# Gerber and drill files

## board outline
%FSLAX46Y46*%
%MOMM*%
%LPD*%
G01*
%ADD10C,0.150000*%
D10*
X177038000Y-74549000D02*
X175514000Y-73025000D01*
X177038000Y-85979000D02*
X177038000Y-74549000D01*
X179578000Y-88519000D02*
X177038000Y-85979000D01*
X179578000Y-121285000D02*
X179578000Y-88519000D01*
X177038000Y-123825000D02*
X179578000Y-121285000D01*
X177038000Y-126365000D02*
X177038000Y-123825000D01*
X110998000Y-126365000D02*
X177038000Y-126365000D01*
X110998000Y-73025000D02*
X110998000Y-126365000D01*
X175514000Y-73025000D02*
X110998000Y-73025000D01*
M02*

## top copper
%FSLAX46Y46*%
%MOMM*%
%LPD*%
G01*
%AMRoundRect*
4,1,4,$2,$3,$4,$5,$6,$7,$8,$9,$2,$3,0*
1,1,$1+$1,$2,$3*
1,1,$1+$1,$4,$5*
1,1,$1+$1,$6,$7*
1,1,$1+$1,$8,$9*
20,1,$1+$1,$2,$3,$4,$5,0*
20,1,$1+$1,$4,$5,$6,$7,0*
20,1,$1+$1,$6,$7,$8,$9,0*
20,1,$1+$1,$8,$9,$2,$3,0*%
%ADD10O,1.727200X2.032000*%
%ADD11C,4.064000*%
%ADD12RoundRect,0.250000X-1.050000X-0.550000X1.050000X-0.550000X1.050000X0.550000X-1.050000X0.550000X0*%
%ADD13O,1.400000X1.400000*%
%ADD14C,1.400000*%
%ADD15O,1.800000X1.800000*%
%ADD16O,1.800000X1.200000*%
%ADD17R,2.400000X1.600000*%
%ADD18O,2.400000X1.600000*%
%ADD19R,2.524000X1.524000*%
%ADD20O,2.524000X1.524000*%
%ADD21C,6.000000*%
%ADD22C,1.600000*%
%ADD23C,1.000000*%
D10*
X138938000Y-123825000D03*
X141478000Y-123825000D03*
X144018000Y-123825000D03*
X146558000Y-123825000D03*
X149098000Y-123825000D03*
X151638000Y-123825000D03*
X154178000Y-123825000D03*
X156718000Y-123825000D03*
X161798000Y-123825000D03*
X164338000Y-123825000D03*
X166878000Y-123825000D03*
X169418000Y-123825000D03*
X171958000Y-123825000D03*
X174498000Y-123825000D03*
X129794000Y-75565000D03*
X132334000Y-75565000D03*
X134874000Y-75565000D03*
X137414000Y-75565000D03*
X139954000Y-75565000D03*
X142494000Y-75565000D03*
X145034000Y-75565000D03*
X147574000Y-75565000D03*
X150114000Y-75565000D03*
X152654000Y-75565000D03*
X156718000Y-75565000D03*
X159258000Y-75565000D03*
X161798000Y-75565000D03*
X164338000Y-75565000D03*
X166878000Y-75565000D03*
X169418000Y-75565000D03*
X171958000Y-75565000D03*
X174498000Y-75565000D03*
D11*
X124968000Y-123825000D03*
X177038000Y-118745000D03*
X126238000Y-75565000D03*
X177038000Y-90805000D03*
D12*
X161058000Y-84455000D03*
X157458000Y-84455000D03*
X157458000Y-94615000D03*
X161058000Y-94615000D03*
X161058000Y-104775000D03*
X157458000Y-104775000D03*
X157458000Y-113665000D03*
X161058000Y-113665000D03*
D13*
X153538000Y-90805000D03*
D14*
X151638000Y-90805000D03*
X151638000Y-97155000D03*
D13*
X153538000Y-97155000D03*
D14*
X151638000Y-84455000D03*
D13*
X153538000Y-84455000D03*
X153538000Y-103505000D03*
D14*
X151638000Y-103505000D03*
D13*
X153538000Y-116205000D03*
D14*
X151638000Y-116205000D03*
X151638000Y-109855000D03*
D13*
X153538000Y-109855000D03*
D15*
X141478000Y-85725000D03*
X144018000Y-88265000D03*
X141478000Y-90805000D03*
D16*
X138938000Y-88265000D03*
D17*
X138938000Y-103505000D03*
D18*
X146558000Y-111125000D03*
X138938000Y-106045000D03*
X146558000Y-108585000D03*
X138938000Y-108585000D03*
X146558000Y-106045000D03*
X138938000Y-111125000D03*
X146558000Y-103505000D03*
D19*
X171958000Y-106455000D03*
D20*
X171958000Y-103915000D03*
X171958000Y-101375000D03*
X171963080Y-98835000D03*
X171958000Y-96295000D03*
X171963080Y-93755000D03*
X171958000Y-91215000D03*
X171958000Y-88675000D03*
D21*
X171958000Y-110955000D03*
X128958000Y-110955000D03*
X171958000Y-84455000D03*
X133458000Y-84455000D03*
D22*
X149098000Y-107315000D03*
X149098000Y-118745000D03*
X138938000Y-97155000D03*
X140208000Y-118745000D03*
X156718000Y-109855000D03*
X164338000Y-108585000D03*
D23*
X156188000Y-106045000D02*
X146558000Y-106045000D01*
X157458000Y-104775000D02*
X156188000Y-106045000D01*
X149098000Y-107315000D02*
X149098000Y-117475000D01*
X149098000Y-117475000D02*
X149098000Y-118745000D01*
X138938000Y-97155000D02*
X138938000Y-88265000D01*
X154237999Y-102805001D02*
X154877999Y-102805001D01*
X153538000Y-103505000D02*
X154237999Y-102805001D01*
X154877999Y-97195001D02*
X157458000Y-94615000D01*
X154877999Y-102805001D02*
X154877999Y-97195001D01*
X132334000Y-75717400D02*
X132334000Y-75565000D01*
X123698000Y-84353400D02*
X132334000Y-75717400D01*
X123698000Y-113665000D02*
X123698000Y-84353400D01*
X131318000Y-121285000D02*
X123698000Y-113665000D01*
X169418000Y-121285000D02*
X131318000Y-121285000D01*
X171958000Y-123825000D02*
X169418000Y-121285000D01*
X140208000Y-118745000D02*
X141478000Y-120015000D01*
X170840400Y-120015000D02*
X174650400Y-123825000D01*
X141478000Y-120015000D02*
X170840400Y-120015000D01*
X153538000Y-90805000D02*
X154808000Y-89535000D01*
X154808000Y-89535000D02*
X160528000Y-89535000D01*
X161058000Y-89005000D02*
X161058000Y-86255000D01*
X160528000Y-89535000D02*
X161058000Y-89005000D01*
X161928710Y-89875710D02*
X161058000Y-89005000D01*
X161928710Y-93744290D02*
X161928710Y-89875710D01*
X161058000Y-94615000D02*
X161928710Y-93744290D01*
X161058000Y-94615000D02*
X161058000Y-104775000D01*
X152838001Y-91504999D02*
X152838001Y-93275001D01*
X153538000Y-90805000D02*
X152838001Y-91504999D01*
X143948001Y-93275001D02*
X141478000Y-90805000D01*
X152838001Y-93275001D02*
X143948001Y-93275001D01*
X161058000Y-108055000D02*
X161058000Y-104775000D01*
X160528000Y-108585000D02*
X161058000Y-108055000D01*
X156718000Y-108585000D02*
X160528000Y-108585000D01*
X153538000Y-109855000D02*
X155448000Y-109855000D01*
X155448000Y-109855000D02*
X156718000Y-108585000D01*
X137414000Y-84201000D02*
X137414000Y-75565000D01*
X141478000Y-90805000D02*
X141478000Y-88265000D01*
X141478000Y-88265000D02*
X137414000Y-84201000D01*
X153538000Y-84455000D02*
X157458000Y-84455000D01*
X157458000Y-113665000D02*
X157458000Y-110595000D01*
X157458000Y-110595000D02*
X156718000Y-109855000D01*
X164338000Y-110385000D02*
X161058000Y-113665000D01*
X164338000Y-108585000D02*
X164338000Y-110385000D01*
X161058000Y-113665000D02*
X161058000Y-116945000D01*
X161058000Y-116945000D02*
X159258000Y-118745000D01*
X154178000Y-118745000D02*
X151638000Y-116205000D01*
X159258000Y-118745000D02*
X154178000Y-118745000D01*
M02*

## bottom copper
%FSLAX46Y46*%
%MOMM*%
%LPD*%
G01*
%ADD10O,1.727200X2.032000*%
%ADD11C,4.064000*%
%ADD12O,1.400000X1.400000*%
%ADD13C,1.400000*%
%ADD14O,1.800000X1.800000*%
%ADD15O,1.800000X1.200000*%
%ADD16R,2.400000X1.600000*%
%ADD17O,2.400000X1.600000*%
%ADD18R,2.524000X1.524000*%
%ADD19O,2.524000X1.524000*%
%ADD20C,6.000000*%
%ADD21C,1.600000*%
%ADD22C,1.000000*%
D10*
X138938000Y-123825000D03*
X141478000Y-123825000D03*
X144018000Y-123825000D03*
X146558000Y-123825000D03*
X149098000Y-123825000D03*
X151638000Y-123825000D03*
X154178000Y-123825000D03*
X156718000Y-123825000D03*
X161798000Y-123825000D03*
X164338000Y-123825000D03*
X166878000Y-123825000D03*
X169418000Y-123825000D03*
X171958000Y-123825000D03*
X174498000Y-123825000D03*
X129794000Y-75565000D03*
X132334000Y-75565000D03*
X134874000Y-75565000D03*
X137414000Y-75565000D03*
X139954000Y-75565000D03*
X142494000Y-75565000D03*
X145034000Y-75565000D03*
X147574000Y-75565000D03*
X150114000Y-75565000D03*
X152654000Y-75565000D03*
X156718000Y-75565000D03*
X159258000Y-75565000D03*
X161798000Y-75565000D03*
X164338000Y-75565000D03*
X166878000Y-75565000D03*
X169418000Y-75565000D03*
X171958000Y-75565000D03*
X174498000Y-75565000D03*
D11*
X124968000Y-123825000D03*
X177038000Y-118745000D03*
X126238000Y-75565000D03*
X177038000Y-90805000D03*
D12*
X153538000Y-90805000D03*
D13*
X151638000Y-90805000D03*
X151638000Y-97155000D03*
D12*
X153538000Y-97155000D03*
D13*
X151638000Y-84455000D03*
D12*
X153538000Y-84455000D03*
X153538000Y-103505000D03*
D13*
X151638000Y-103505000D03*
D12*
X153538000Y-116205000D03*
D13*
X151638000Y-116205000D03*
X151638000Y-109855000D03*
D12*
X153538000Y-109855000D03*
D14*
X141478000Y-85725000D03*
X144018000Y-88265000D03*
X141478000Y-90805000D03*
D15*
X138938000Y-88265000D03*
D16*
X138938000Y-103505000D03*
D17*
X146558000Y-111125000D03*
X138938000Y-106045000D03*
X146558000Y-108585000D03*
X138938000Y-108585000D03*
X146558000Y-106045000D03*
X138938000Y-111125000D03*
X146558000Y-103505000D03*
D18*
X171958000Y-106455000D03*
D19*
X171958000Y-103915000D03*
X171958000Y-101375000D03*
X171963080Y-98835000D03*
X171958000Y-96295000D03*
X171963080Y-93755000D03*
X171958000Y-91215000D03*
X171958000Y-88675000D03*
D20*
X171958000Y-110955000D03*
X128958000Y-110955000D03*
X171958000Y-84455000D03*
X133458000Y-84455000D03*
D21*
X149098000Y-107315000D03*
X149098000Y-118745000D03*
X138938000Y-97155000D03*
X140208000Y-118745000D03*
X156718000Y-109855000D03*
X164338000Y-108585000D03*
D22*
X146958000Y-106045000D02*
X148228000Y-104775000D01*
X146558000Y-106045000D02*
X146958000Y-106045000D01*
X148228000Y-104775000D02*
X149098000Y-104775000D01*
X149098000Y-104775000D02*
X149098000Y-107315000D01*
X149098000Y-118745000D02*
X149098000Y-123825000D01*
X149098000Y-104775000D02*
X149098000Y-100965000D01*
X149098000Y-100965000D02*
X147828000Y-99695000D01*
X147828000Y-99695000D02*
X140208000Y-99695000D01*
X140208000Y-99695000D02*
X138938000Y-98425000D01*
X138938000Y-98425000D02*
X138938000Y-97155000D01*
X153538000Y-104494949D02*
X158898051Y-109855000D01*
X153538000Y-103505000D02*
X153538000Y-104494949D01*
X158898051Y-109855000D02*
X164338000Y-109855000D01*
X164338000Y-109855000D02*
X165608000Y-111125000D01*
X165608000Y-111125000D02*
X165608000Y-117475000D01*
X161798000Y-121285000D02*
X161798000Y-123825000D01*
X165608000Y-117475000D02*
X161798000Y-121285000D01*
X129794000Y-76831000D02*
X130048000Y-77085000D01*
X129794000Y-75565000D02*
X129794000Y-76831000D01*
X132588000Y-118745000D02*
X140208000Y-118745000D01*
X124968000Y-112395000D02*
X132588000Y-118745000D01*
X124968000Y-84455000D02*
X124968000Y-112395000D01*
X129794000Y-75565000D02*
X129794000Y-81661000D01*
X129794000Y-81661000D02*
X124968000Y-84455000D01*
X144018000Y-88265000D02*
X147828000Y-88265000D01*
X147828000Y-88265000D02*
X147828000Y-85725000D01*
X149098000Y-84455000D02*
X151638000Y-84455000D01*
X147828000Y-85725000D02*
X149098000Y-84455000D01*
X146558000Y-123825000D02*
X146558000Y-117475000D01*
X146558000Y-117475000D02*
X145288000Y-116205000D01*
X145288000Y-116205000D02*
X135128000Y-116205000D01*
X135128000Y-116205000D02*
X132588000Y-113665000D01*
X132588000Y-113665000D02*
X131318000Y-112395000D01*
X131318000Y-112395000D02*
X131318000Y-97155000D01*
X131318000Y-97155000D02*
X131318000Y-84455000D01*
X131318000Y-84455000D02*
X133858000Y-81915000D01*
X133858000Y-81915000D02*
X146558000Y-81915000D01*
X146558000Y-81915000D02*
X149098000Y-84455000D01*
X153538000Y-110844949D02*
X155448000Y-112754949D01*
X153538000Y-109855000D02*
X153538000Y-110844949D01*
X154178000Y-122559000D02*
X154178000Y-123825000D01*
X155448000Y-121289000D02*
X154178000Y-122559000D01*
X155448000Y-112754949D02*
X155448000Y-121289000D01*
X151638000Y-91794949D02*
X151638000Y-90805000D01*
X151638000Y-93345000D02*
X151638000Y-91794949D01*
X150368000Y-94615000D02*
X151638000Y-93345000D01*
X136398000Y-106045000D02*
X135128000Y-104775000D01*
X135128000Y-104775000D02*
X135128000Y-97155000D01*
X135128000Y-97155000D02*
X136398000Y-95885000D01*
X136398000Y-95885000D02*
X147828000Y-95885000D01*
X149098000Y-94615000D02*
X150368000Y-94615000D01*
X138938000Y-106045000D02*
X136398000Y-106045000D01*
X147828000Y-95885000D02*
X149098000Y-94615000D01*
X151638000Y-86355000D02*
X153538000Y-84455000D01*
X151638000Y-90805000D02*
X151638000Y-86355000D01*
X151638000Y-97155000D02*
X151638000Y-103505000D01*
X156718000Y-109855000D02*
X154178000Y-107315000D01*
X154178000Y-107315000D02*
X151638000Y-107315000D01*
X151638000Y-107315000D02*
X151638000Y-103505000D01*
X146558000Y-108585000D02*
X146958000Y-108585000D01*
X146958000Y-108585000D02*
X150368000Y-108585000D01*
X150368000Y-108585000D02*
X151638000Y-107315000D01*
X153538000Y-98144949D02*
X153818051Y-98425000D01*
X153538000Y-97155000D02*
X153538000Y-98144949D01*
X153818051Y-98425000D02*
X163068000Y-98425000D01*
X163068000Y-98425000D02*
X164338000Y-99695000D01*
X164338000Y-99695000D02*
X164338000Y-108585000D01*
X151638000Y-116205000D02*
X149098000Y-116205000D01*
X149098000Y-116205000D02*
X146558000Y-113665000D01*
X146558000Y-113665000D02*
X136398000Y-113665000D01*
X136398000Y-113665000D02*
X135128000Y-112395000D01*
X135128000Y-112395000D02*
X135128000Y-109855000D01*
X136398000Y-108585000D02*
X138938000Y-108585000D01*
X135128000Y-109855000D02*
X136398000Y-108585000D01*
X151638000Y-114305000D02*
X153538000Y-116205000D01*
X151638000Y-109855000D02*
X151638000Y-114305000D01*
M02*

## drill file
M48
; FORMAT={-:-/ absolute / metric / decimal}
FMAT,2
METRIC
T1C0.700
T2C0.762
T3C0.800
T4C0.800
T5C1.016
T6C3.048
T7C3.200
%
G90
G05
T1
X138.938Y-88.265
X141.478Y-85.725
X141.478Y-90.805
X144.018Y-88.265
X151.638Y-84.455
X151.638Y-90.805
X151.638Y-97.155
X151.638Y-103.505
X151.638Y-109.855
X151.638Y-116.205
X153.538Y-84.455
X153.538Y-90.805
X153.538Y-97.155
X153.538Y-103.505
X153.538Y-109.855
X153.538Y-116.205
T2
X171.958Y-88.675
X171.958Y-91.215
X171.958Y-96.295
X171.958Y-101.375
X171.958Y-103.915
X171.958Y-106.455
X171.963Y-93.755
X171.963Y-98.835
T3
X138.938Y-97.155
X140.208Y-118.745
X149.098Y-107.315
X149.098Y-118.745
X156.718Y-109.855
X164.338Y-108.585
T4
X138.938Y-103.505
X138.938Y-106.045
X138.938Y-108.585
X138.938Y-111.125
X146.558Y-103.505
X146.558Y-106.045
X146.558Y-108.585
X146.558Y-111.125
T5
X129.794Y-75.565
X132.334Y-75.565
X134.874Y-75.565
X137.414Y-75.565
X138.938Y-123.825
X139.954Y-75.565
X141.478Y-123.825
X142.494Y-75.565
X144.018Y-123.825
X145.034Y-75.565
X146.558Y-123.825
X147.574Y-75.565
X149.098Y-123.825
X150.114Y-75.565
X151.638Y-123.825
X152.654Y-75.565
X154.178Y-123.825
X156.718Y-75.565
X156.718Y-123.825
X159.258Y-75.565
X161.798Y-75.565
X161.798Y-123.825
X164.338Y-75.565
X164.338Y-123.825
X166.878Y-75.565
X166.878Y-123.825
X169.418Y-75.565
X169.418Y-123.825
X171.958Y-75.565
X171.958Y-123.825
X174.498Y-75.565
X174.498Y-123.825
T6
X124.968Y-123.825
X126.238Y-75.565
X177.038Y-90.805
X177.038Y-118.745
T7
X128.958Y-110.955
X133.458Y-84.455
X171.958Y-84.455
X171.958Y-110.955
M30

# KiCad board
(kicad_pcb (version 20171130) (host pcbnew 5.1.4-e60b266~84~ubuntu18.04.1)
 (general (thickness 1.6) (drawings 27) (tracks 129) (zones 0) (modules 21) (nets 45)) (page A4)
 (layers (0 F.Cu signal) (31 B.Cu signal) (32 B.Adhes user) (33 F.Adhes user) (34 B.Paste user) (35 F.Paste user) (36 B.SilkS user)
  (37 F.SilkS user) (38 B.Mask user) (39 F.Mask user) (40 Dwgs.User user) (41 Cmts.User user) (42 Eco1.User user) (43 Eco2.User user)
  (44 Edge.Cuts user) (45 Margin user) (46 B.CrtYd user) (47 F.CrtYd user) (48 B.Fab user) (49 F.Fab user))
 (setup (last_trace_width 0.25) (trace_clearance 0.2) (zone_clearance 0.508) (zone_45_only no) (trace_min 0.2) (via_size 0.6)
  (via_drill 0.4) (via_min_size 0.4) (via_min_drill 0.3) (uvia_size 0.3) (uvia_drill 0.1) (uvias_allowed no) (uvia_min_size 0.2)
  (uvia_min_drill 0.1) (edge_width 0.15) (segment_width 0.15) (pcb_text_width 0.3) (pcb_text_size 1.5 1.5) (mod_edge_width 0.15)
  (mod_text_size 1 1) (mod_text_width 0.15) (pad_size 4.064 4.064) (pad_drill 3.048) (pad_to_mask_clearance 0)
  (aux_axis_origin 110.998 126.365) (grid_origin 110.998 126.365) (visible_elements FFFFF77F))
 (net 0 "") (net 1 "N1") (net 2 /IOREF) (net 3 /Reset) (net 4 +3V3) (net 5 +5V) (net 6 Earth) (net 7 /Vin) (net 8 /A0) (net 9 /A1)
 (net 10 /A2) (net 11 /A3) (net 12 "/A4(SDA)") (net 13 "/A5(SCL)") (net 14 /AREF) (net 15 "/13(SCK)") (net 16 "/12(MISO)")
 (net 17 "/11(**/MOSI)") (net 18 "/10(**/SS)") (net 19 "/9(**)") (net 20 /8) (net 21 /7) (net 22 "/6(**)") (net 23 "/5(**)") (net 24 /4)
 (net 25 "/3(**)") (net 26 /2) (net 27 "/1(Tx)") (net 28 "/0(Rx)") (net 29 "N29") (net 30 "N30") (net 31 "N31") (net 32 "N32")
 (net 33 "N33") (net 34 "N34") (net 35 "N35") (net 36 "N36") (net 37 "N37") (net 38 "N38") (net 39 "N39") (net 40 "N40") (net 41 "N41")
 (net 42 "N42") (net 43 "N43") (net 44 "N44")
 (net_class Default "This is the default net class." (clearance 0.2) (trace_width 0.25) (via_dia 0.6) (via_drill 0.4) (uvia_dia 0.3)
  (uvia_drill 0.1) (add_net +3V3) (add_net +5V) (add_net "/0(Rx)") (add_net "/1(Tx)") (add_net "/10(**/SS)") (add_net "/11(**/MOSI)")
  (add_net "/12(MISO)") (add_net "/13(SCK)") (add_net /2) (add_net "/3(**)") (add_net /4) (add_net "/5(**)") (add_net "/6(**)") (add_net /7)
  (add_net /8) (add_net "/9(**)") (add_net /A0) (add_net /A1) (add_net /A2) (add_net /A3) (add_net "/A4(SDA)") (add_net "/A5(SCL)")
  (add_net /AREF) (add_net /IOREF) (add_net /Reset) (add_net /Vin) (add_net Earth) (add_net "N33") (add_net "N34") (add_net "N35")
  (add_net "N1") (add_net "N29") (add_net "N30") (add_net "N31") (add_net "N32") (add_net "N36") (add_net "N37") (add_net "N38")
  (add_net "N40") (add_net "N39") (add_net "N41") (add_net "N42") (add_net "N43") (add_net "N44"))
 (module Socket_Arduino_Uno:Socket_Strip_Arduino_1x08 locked (layer F.Cu) (at 138.938 123.825)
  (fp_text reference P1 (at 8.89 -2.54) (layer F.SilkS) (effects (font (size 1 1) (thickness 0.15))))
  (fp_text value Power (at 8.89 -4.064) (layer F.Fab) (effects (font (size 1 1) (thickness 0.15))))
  (pad 1 thru_hole oval (at 0 0) (size 1.7272 2.032) (drill 1.016) (layers *.Cu *.Mask F.SilkS) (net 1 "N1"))
  (pad 2 thru_hole oval (at 2.54 0) (size 1.7272 2.032) (drill 1.016) (layers *.Cu *.Mask F.SilkS) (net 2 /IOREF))
  (pad 3 thru_hole oval (at 5.08 0) (size 1.7272 2.032) (drill 1.016) (layers *.Cu *.Mask F.SilkS) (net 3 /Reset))
  (pad 4 thru_hole oval (at 7.62 0) (size 1.7272 2.032) (drill 1.016) (layers *.Cu *.Mask F.SilkS) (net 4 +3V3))
  (pad 5 thru_hole oval (at 10.16 0) (size 1.7272 2.032) (drill 1.016) (layers *.Cu *.Mask F.SilkS) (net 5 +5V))
  (pad 6 thru_hole oval (at 12.7 0) (size 1.7272 2.032) (drill 1.016) (layers *.Cu *.Mask F.SilkS) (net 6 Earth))
  (pad 7 thru_hole oval (at 15.24 0) (size 1.7272 2.032) (drill 1.016) (layers *.Cu *.Mask F.SilkS) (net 6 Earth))
  (pad 8 thru_hole oval (at 17.78 0) (size 1.7272 2.032) (drill 1.016) (layers *.Cu *.Mask F.SilkS) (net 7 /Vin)))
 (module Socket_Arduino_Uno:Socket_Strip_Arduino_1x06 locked (layer F.Cu) (at 161.798 123.825)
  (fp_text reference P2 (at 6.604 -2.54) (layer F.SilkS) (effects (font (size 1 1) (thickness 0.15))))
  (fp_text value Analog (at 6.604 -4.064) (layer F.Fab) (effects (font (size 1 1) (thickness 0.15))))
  (pad 1 thru_hole oval (at 0 0) (size 1.7272 2.032) (drill 1.016) (layers *.Cu *.Mask F.SilkS) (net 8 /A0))
  (pad 2 thru_hole oval (at 2.54 0) (size 1.7272 2.032) (drill 1.016) (layers *.Cu *.Mask F.SilkS) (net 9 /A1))
  (pad 3 thru_hole oval (at 5.08 0) (size 1.7272 2.032) (drill 1.016) (layers *.Cu *.Mask F.SilkS) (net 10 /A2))
  (pad 4 thru_hole oval (at 7.62 0) (size 1.7272 2.032) (drill 1.016) (layers *.Cu *.Mask F.SilkS) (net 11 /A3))
  (pad 5 thru_hole oval (at 10.16 0) (size 1.7272 2.032) (drill 1.016) (layers *.Cu *.Mask F.SilkS) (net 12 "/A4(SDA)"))
  (pad 6 thru_hole oval (at 12.7 0) (size 1.7272 2.032) (drill 1.016) (layers *.Cu *.Mask F.SilkS) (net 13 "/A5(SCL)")))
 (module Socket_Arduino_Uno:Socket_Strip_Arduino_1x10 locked (layer F.Cu) (at 129.794 75.565)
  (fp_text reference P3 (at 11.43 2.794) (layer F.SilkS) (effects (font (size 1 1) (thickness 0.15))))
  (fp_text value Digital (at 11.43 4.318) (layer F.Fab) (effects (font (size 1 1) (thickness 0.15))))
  (pad 1 thru_hole oval (at 0 0) (size 1.7272 2.032) (drill 1.016) (layers *.Cu *.Mask F.SilkS) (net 13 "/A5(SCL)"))
  (pad 2 thru_hole oval (at 2.54 0) (size 1.7272 2.032) (drill 1.016) (layers *.Cu *.Mask F.SilkS) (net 12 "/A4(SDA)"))
  (pad 3 thru_hole oval (at 5.08 0) (size 1.7272 2.032) (drill 1.016) (layers *.Cu *.Mask F.SilkS) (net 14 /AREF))
  (pad 4 thru_hole oval (at 7.62 0) (size 1.7272 2.032) (drill 1.016) (layers *.Cu *.Mask F.SilkS) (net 6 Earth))
  (pad 5 thru_hole oval (at 10.16 0) (size 1.7272 2.032) (drill 1.016) (layers *.Cu *.Mask F.SilkS) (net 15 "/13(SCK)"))
  (pad 6 thru_hole oval (at 12.7 0) (size 1.7272 2.032) (drill 1.016) (layers *.Cu *.Mask F.SilkS) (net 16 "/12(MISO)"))
  (pad 7 thru_hole oval (at 15.24 0) (size 1.7272 2.032) (drill 1.016) (layers *.Cu *.Mask F.SilkS) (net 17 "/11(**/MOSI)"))
  (pad 8 thru_hole oval (at 17.78 0) (size 1.7272 2.032) (drill 1.016) (layers *.Cu *.Mask F.SilkS) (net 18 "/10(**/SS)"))
  (pad 9 thru_hole oval (at 20.32 0) (size 1.7272 2.032) (drill 1.016) (layers *.Cu *.Mask F.SilkS) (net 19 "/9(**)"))
  (pad 10 thru_hole oval (at 22.86 0) (size 1.7272 2.032) (drill 1.016) (layers *.Cu *.Mask F.SilkS) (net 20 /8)))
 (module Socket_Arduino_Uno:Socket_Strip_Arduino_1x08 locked (layer F.Cu) (at 156.718 75.565)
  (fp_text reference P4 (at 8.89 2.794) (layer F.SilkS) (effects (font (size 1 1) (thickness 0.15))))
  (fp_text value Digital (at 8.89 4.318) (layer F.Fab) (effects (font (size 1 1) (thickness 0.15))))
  (pad 1 thru_hole oval (at 0 0) (size 1.7272 2.032) (drill 1.016) (layers *.Cu *.Mask F.SilkS) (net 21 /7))
  (pad 2 thru_hole oval (at 2.54 0) (size 1.7272 2.032) (drill 1.016) (layers *.Cu *.Mask F.SilkS) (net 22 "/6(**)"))
  (pad 3 thru_hole oval (at 5.08 0) (size 1.7272 2.032) (drill 1.016) (layers *.Cu *.Mask F.SilkS) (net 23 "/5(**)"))
  (pad 4 thru_hole oval (at 7.62 0) (size 1.7272 2.032) (drill 1.016) (layers *.Cu *.Mask F.SilkS) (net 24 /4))
  (pad 5 thru_hole oval (at 10.16 0) (size 1.7272 2.032) (drill 1.016) (layers *.Cu *.Mask F.SilkS) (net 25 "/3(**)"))
  (pad 6 thru_hole oval (at 12.7 0) (size 1.7272 2.032) (drill 1.016) (layers *.Cu *.Mask F.SilkS) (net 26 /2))
  (pad 7 thru_hole oval (at 15.24 0) (size 1.7272 2.032) (drill 1.016) (layers *.Cu *.Mask F.SilkS) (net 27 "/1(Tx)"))
  (pad 8 thru_hole oval (at 17.78 0) (size 1.7272 2.032) (drill 1.016) (layers *.Cu *.Mask F.SilkS) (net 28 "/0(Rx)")))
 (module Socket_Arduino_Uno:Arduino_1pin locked (layer F.Cu) (at 124.968 123.825)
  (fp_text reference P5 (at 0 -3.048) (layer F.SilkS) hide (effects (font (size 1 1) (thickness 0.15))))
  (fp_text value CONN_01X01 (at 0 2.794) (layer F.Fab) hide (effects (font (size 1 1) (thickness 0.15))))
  (pad 1 thru_hole circle (at 0 0) (size 4.064 4.064) (drill 3.048) (layers *.Cu *.Mask F.SilkS) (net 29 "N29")))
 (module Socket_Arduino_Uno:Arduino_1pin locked (layer F.Cu) (at 177.038 118.745)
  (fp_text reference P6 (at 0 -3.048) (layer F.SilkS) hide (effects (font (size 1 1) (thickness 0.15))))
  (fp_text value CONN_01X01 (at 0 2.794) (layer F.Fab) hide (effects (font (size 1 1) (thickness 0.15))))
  (pad 1 thru_hole circle (at 0 0) (size 4.064 4.064) (drill 3.048) (layers *.Cu *.Mask F.SilkS) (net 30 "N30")))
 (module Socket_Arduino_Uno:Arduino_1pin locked (layer F.Cu) (at 126.238 75.565)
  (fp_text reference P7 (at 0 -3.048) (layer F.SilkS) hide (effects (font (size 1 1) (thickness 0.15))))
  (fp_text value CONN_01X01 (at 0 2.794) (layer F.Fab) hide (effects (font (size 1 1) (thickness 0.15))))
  (pad 1 thru_hole circle (at 0 0) (size 4.064 4.064) (drill 3.048) (layers *.Cu *.Mask F.SilkS) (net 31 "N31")))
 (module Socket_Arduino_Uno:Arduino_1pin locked (layer F.Cu) (at 177.038 90.805)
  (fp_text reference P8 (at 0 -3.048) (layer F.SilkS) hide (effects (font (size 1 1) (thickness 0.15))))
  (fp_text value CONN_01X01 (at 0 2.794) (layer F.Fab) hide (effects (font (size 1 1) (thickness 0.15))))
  (pad 1 thru_hole circle (at 0 0) (size 4.064 4.064) (drill 3.048) (layers *.Cu *.Mask F.SilkS) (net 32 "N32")))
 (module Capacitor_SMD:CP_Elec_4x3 (layer F.Cu) (at 159.258 84.455)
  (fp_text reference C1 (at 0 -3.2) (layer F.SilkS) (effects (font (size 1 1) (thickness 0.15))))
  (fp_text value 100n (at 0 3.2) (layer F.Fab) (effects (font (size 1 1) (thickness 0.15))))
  (pad 2 smd roundrect (at 1.8 0) (size 2.6 1.6) (layers F.Cu F.Paste F.Mask) (roundrect_rratio 0.15625) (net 6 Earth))
  (pad 1 smd roundrect (at -1.8 0) (size 2.6 1.6) (layers F.Cu F.Paste F.Mask) (roundrect_rratio 0.15625) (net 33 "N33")))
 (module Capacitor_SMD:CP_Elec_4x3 (layer F.Cu) (at 159.258 94.615)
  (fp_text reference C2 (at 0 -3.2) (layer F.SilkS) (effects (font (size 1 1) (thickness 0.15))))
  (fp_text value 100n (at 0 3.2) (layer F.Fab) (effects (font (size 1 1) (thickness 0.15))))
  (pad 1 smd roundrect (at -1.8 0) (size 2.6 1.6) (layers F.Cu F.Paste F.Mask) (roundrect_rratio 0.15625) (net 8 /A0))
  (pad 2 smd roundrect (at 1.8 0) (size 2.6 1.6) (layers F.Cu F.Paste F.Mask) (roundrect_rratio 0.15625) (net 6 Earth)))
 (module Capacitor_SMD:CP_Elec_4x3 (layer F.Cu) (at 159.258 104.775)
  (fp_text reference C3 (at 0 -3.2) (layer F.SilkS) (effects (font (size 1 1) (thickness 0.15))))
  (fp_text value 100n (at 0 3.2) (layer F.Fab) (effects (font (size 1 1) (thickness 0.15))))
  (pad 2 smd roundrect (at 1.8 0) (size 2.6 1.6) (layers F.Cu F.Paste F.Mask) (roundrect_rratio 0.15625) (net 6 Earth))
  (pad 1 smd roundrect (at -1.8 0) (size 2.6 1.6) (layers F.Cu F.Paste F.Mask) (roundrect_rratio 0.15625) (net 5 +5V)))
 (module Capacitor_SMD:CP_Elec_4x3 (layer F.Cu) (at 159.258 113.665)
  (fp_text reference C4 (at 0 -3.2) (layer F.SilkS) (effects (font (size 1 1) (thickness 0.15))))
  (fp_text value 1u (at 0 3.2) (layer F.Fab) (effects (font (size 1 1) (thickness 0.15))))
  (pad 1 smd roundrect (at -1.8 0) (size 2.6 1.6) (layers F.Cu F.Paste F.Mask) (roundrect_rratio 0.15625) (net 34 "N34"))
  (pad 2 smd roundrect (at 1.8 0) (size 2.6 1.6) (layers F.Cu F.Paste F.Mask) (roundrect_rratio 0.15625) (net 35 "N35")))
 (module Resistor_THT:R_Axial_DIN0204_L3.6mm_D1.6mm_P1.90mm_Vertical (layer F.Cu) (at 151.638 90.805)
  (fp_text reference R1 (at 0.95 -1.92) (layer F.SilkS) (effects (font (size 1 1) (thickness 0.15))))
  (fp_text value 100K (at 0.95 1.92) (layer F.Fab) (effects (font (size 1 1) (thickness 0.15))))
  (pad 2 thru_hole oval (at 1.9 0) (size 1.4 1.4) (drill 0.7) (layers *.Cu *.Mask) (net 6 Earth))
  (pad 1 thru_hole circle (at 0 0) (size 1.4 1.4) (drill 0.7) (layers *.Cu *.Mask) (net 33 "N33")))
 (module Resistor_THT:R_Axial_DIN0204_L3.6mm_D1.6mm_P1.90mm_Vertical (layer F.Cu) (at 151.638 97.155)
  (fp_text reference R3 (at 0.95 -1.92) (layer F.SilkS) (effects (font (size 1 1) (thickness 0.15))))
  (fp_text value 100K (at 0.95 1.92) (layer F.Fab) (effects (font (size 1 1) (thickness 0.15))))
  (pad 1 thru_hole circle (at 0 0) (size 1.4 1.4) (drill 0.7) (layers *.Cu *.Mask) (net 34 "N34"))
  (pad 2 thru_hole oval (at 1.9 0) (size 1.4 1.4) (drill 0.7) (layers *.Cu *.Mask) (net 35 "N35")))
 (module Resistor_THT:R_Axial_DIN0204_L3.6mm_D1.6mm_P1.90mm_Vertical (layer F.Cu) (at 151.638 84.455)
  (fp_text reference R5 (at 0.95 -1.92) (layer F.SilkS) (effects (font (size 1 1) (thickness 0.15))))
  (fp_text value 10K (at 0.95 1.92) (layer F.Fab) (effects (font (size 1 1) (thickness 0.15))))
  (pad 1 thru_hole circle (at 0 0) (size 1.4 1.4) (drill 0.7) (layers *.Cu *.Mask) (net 4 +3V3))
  (pad 2 thru_hole oval (at 1.9 0) (size 1.4 1.4) (drill 0.7) (layers *.Cu *.Mask) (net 33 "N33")))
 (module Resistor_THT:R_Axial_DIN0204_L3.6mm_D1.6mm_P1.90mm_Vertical (layer F.Cu) (at 151.638 103.505)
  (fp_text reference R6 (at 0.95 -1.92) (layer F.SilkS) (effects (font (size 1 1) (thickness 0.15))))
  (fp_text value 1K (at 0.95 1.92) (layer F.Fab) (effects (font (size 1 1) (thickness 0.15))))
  (pad 2 thru_hole oval (at 1.9 0) (size 1.4 1.4) (drill 0.7) (layers *.Cu *.Mask) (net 8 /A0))
  (pad 1 thru_hole circle (at 0 0) (size 1.4 1.4) (drill 0.7) (layers *.Cu *.Mask) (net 34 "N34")))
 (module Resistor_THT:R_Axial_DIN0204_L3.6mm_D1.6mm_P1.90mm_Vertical (layer F.Cu) (at 151.638 116.205)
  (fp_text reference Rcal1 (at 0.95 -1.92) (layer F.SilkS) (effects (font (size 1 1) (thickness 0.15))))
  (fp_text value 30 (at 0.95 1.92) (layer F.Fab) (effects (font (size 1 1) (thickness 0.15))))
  (pad 2 thru_hole oval (at 1.9 0) (size 1.4 1.4) (drill 0.7) (layers *.Cu *.Mask) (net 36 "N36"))
  (pad 1 thru_hole circle (at 0 0) (size 1.4 1.4) (drill 0.7) (layers *.Cu *.Mask) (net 35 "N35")))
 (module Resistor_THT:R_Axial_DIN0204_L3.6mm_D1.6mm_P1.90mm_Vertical (layer F.Cu) (at 151.638 109.855)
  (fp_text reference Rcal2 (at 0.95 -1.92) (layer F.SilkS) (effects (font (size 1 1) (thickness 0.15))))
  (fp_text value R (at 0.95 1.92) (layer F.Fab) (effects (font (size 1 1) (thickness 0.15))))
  (pad 1 thru_hole circle (at 0 0) (size 1.4 1.4) (drill 0.7) (layers *.Cu *.Mask) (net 36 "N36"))
  (pad 2 thru_hole oval (at 1.9 0) (size 1.4 1.4) (drill 0.7) (layers *.Cu *.Mask) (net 6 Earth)))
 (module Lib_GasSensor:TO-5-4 (layer F.Cu) (at 138.938 88.265)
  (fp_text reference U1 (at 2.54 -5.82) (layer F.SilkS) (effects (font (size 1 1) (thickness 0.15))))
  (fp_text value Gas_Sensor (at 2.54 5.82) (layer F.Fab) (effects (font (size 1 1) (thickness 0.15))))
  (pad 4 thru_hole oval (at 2.54 -2.54) (size 1.8 1.8) (drill 0.7) (layers *.Cu *.Mask) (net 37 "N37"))
  (pad 3 thru_hole oval (at 5.08 0) (size 1.8 1.8) (drill 0.7) (layers *.Cu *.Mask) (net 4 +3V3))
  (pad 2 thru_hole oval (at 2.54 2.54) (size 1.8 1.8) (drill 0.7) (layers *.Cu *.Mask) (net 6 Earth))
  (pad 1 thru_hole oval (at 0 0) (size 1.8 1.2) (drill 0.7) (layers *.Cu *.Mask) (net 5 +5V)))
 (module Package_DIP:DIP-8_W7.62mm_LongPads (layer F.Cu) (at 138.938 103.505)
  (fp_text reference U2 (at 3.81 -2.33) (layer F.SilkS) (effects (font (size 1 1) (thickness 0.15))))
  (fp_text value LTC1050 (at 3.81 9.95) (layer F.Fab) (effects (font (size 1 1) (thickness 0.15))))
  (pad 1 thru_hole rect (at 0 0) (size 2.4 1.6) (drill 0.8) (layers *.Cu *.Mask) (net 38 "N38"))
  (pad 5 thru_hole oval (at 7.62 7.62) (size 2.4 1.6) (drill 0.8) (layers *.Cu *.Mask) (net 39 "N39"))
  (pad 2 thru_hole oval (at 0 2.54) (size 2.4 1.6) (drill 0.8) (layers *.Cu *.Mask) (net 33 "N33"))
  (pad 6 thru_hole oval (at 7.62 5.08) (size 2.4 1.6) (drill 0.8) (layers *.Cu *.Mask) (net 34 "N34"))
  (pad 3 thru_hole oval (at 0 5.08) (size 2.4 1.6) (drill 0.8) (layers *.Cu *.Mask) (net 35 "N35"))
  (pad 7 thru_hole oval (at 7.62 2.54) (size 2.4 1.6) (drill 0.8) (layers *.Cu *.Mask) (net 5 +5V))
  (pad 4 thru_hole oval (at 0 7.62) (size 2.4 1.6) (drill 0.8) (layers *.Cu *.Mask) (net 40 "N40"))
  (pad 8 thru_hole oval (at 7.62 0) (size 2.4 1.6) (drill 0.8) (layers *.Cu *.Mask) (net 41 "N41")))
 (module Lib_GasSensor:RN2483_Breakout (layer F.Cu) (at 171.958 106.455 90)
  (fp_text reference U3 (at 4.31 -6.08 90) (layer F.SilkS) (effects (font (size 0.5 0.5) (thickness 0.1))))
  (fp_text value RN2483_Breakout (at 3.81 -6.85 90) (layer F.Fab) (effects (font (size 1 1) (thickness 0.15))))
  (pad 1 thru_hole rect (at 0 0 90) (size 1.524 2.524) (drill 0.762) (layers *.Cu *.Mask) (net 18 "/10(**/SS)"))
  (pad 2 thru_hole oval (at 2.54 0 90) (size 1.524 2.524) (drill 0.762) (layers *.Cu *.Mask) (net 17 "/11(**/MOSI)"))
  (pad 3 thru_hole oval (at 5.08 0 90) (size 1.524 2.524) (drill 0.762) (layers *.Cu *.Mask) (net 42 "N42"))
  (pad 4 thru_hole oval (at 7.62 0.00508 90) (size 1.524 2.524) (drill 0.762) (layers *.Cu *.Mask) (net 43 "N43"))
  (pad 5 thru_hole oval (at 10.16 0 90) (size 1.524 2.524) (drill 0.762) (layers *.Cu *.Mask) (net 16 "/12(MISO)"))
  (pad 6 thru_hole oval (at 12.7 0.00508 90) (size 1.524 2.524) (drill 0.762) (layers *.Cu *.Mask) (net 4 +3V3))
  (pad 7 thru_hole oval (at 15.24 0 90) (size 1.524 2.524) (drill 0.762) (layers *.Cu *.Mask) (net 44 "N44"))
  (pad 8 thru_hole oval (at 17.78 0 90) (size 1.524 2.524) (drill 0.762) (layers *.Cu *.Mask) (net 6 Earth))
  (pad "" thru_hole circle (at -4.5 0 90) (size 6 6) (drill 3.2) (layers *.Cu *.Mask))
  (pad "" thru_hole circle (at -4.5 -43 90) (size 6 6) (drill 3.2) (layers *.Cu *.Mask))
  (pad "" thru_hole circle (at 22 0 90) (size 6 6) (drill 3.2) (layers *.Cu *.Mask))
  (pad "" thru_hole circle (at 22 -38.5 90) (size 6 6) (drill 3.2) (layers *.Cu *.Mask)))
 (gr_line (start 177.038 74.549) (end 175.514 73.025) (angle 90) (layer Edge.Cuts) (width 0.15))
 (gr_line (start 177.038 85.979) (end 177.038 74.549) (angle 90) (layer Edge.Cuts) (width 0.15))
 (gr_line (start 179.578 88.519) (end 177.038 85.979) (angle 90) (layer Edge.Cuts) (width 0.15))
 (gr_line (start 179.578 121.285) (end 179.578 88.519) (angle 90) (layer Edge.Cuts) (width 0.15))
 (gr_line (start 177.038 123.825) (end 179.578 121.285) (angle 90) (layer Edge.Cuts) (width 0.15))
 (gr_line (start 177.038 126.365) (end 177.038 123.825) (angle 90) (layer Edge.Cuts) (width 0.15))
 (gr_line (start 110.998 126.365) (end 177.038 126.365) (angle 90) (layer Edge.Cuts) (width 0.15))
 (gr_line (start 110.998 73.025) (end 110.998 126.365) (angle 90) (layer Edge.Cuts) (width 0.15))
 (gr_line (start 175.514 73.025) (end 110.998 73.025) (angle 90) (layer Edge.Cuts) (width 0.15))
 (segment (start 156.188 106.045) (end 146.558 106.045) (width 1) (layer F.Cu) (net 5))
 (segment (start 157.458 104.775) (end 156.188 106.045) (width 1) (layer F.Cu) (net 5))
 (segment (start 146.958 106.045) (end 148.228 104.775) (width 1) (layer B.Cu) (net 5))
 (segment (start 146.558 106.045) (end 146.958 106.045) (width 1) (layer B.Cu) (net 5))
 (segment (start 148.228 104.775) (end 149.098 104.775) (width 1) (layer B.Cu) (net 5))
 (via (at 149.098 107.315) (size 1.6) (drill 0.8) (layers F.Cu B.Cu) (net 5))
 (segment (start 149.098 104.775) (end 149.098 107.315) (width 1) (layer B.Cu) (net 5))
 (segment (start 149.098 107.315) (end 149.098 117.475) (width 1) (layer F.Cu) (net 5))
 (via (at 149.098 118.745) (size 1.6) (drill 0.8) (layers F.Cu B.Cu) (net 5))
 (segment (start 149.098 117.475) (end 149.098 118.745) (width 1) (layer F.Cu) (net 5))
 (segment (start 149.098 118.745) (end 149.098 123.825) (width 1) (layer B.Cu) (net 5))
 (segment (start 149.098 104.775) (end 149.098 100.965) (width 1) (layer B.Cu) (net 5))
 (segment (start 149.098 100.965) (end 147.828 99.695) (width 1) (layer B.Cu) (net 5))
 (segment (start 147.828 99.695) (end 140.208 99.695) (width 1) (layer B.Cu) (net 5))
 (via (at 138.938 97.155) (size 1.6) (drill 0.8) (layers F.Cu B.Cu) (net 5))
 (segment (start 140.208 99.695) (end 138.938 98.425) (width 1) (layer B.Cu) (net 5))
 (segment (start 138.938 98.425) (end 138.938 97.155) (width 1) (layer B.Cu) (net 5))
 (segment (start 138.938 97.155) (end 138.938 88.265) (width 1) (layer F.Cu) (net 5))
 (segment (start 154.237999 102.805001) (end 154.877999 102.805001) (width 1) (layer F.Cu) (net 8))
 (segment (start 153.538 103.505) (end 154.237999 102.805001) (width 1) (layer F.Cu) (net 8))
 (segment (start 154.877999 97.195001) (end 157.458 94.615) (width 1) (layer F.Cu) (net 8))
 (segment (start 154.877999 102.805001) (end 154.877999 97.195001) (width 1) (layer F.Cu) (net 8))
 (segment (start 153.538 104.494949) (end 158.898051 109.855) (width 1) (layer B.Cu) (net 8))
 (segment (start 153.538 103.505) (end 153.538 104.494949) (width 1) (layer B.Cu) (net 8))
 (segment (start 158.898051 109.855) (end 164.338 109.855) (width 1) (layer B.Cu) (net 8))
 (segment (start 164.338 109.855) (end 165.608 111.125) (width 1) (layer B.Cu) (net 8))
 (segment (start 165.608 111.125) (end 165.608 117.475) (width 1) (layer B.Cu) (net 8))
 (segment (start 161.798 121.285) (end 161.798 123.825) (width 1) (layer B.Cu) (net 8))
 (segment (start 165.608 117.475) (end 161.798 121.285) (width 1) (layer B.Cu) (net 8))
 (segment (start 132.334 75.7174) (end 132.334 75.565) (width 1) (layer F.Cu) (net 12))
 (segment (start 123.698 84.3534) (end 132.334 75.7174) (width 1) (layer F.Cu) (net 12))
 (segment (start 123.698 113.665) (end 123.698 84.3534) (width 1) (layer F.Cu) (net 12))
 (segment (start 131.318 121.285) (end 123.698 113.665) (width 1) (layer F.Cu) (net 12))
 (segment (start 169.418 121.285) (end 131.318 121.285) (width 1) (layer F.Cu) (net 12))
 (segment (start 171.958 123.825) (end 169.418 121.285) (width 1) (layer F.Cu) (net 12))
 (segment (start 129.794 76.831) (end 130.048 77.085) (width 1) (layer B.Cu) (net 13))
 (segment (start 129.794 75.565) (end 129.794 76.831) (width 1) (layer B.Cu) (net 13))
 (via (at 140.208 118.745) (size 1.6) (drill 0.8) (layers F.Cu B.Cu) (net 13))
 (segment (start 140.208 118.745) (end 141.478 120.015) (width 1) (layer F.Cu) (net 13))
 (segment (start 170.8404 120.015) (end 174.6504 123.825) (width 1) (layer F.Cu) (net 13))
 (segment (start 141.478 120.015) (end 170.8404 120.015) (width 1) (layer F.Cu) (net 13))
 (segment (start 132.588 118.745) (end 140.208 118.745) (width 1) (layer B.Cu) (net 13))
 (segment (start 124.968 112.395) (end 132.588 118.745) (width 1) (layer B.Cu) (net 13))
 (segment (start 124.968 84.455) (end 124.968 112.395) (width 1) (layer B.Cu) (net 13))
 (segment (start 129.794 75.565) (end 129.794 81.661) (width 1) (layer B.Cu) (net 13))
 (segment (start 129.794 81.661) (end 124.968 84.455) (width 1) (layer B.Cu) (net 13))
 (segment (start 144.018 88.265) (end 147.828 88.265) (width 1) (layer B.Cu) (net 4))
 (segment (start 147.828 88.265) (end 147.828 85.725) (width 1) (layer B.Cu) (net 4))
 (segment (start 149.098 84.455) (end 151.638 84.455) (width 1) (layer B.Cu) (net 4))
 (segment (start 147.828 85.725) (end 149.098 84.455) (width 1) (layer B.Cu) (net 4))
 (segment (start 146.558 123.825) (end 146.558 117.475) (width 1) (layer B.Cu) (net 4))
 (segment (start 146.558 117.475) (end 145.288 116.205) (width 1) (layer B.Cu) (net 4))
 (segment (start 145.288 116.205) (end 135.128 116.205) (width 1) (layer B.Cu) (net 4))
 (segment (start 135.128 116.205) (end 132.588 113.665) (width 1) (layer B.Cu) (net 4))
 (segment (start 132.588 113.665) (end 131.318 112.395) (width 1) (layer B.Cu) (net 4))
 (segment (start 131.318 112.395) (end 131.318 97.155) (width 1) (layer B.Cu) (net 4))
 (segment (start 131.318 97.155) (end 131.318 84.455) (width 1) (layer B.Cu) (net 4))
 (segment (start 131.318 84.455) (end 133.858 81.915) (width 1) (layer B.Cu) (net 4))
 (segment (start 133.858 81.915) (end 146.558 81.915) (width 1) (layer B.Cu) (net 4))
 (segment (start 146.558 81.915) (end 149.098 84.455) (width 1) (layer B.Cu) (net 4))
 (segment (start 153.538 90.805) (end 154.808 89.535) (width 1) (layer F.Cu) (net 6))
 (segment (start 154.808 89.535) (end 160.528 89.535) (width 1) (layer F.Cu) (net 6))
 (segment (start 161.058 89.005) (end 161.058 86.255) (width 1) (layer F.Cu) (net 6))
 (segment (start 160.528 89.535) (end 161.058 89.005) (width 1) (layer F.Cu) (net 6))
 (segment (start 161.92871 89.87571) (end 161.058 89.005) (width 1) (layer F.Cu) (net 6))
 (segment (start 161.92871 93.74429) (end 161.92871 89.87571) (width 1) (layer F.Cu) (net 6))
 (segment (start 161.058 94.615) (end 161.92871 93.74429) (width 1) (layer F.Cu) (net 6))
 (segment (start 161.058 94.615) (end 161.058 104.775) (width 1) (layer F.Cu) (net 6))
 (segment (start 152.838001 91.504999) (end 152.838001 93.275001) (width 1) (layer F.Cu) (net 6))
 (segment (start 153.538 90.805) (end 152.838001 91.504999) (width 1) (layer F.Cu) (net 6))
 (segment (start 143.948001 93.275001) (end 141.478 90.805) (width 1) (layer F.Cu) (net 6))
 (segment (start 152.838001 93.275001) (end 143.948001 93.275001) (width 1) (layer F.Cu) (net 6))
 (segment (start 153.538 110.844949) (end 155.448 112.754949) (width 1) (layer B.Cu) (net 6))
 (segment (start 153.538 109.855) (end 153.538 110.844949) (width 1) (layer B.Cu) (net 6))
 (segment (start 154.178 122.559) (end 154.178 123.825) (width 1) (layer B.Cu) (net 6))
 (segment (start 155.448 121.289) (end 154.178 122.559) (width 1) (layer B.Cu) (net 6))
 (segment (start 155.448 112.754949) (end 155.448 121.289) (width 1) (layer B.Cu) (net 6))
 (segment (start 161.058 108.055) (end 161.058 104.775) (width 1) (layer F.Cu) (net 6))
 (segment (start 160.528 108.585) (end 161.058 108.055) (width 1) (layer F.Cu) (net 6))
 (segment (start 156.718 108.585) (end 160.528 108.585) (width 1) (layer F.Cu) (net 6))
 (segment (start 153.538 109.855) (end 155.448 109.855) (width 1) (layer F.Cu) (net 6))
 (segment (start 155.448 109.855) (end 156.718 108.585) (width 1) (layer F.Cu) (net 6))
 (segment (start 137.414 84.201) (end 137.414 75.565) (width 1) (layer F.Cu) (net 6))
 (segment (start 141.478 90.805) (end 141.478 88.265) (width 1) (layer F.Cu) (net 6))
 (segment (start 141.478 88.265) (end 137.414 84.201) (width 1) (layer F.Cu) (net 6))
 (segment (start 151.638 91.794949) (end 151.638 90.805) (width 1) (layer B.Cu) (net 33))
 (segment (start 151.638 93.345) (end 151.638 91.794949) (width 1) (layer B.Cu) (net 33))
 (segment (start 150.368 94.615) (end 151.638 93.345) (width 1) (layer B.Cu) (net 33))
 (segment (start 136.398 106.045) (end 135.128 104.775) (width 1) (layer B.Cu) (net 33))
 (segment (start 135.128 104.775) (end 135.128 97.155) (width 1) (layer B.Cu) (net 33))
 (segment (start 135.128 97.155) (end 136.398 95.885) (width 1) (layer B.Cu) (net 33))
 (segment (start 136.398 95.885) (end 147.828 95.885) (width 1) (layer B.Cu) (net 33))
 (segment (start 149.098 94.615) (end 150.368 94.615) (width 1) (layer B.Cu) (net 33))
 (segment (start 138.938 106.045) (end 136.398 106.045) (width 1) (layer B.Cu) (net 33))
 (segment (start 147.828 95.885) (end 149.098 94.615) (width 1) (layer B.Cu) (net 33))
 (segment (start 153.538 84.455) (end 157.458 84.455) (width 1) (layer F.Cu) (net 33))
 (segment (start 151.638 86.355) (end 153.538 84.455) (width 1) (layer B.Cu) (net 33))
 (segment (start 151.638 90.805) (end 151.638 86.355) (width 1) (layer B.Cu) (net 33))
 (segment (start 151.638 97.155) (end 151.638 103.505) (width 1) (layer B.Cu) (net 34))
 (via (at 156.718 109.855) (size 1.6) (drill 0.8) (layers F.Cu B.Cu) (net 34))
 (segment (start 157.458 113.665) (end 157.458 110.595) (width 1) (layer F.Cu) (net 34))
 (segment (start 157.458 110.595) (end 156.718 109.855) (width 1) (layer F.Cu) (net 34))
 (segment (start 156.718 109.855) (end 154.178 107.315) (width 1) (layer B.Cu) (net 34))
 (segment (start 154.178 107.315) (end 151.638 107.315) (width 1) (layer B.Cu) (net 34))
 (segment (start 151.638 107.315) (end 151.638 103.505) (width 1) (layer B.Cu) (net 34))
 (segment (start 146.558 108.585) (end 146.958 108.585) (width 1) (layer B.Cu) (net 34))
 (segment (start 146.958 108.585) (end 150.368 108.585) (width 1) (layer B.Cu) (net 34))
 (segment (start 150.368 108.585) (end 151.638 107.315) (width 1) (layer B.Cu) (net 34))
 (segment (start 153.538 98.144949) (end 153.818051 98.425) (width 1) (layer B.Cu) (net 35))
 (segment (start 153.538 97.155) (end 153.538 98.144949) (width 1) (layer B.Cu) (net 35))
 (segment (start 153.818051 98.425) (end 163.068 98.425) (width 1) (layer B.Cu) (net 35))
 (segment (start 163.068 98.425) (end 164.338 99.695) (width 1) (layer B.Cu) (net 35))
 (via (at 164.338 108.585) (size 1.6) (drill 0.8) (layers F.Cu B.Cu) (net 35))
 (segment (start 164.338 99.695) (end 164.338 108.585) (width 1) (layer B.Cu) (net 35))
 (segment (start 164.338 110.385) (end 161.058 113.665) (width 1) (layer F.Cu) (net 35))
 (segment (start 164.338 108.585) (end 164.338 110.385) (width 1) (layer F.Cu) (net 35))
 (segment (start 161.058 113.665) (end 161.058 116.945) (width 1) (layer F.Cu) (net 35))
 (segment (start 161.058 116.945) (end 159.258 118.745) (width 1) (layer F.Cu) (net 35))
 (segment (start 154.178 118.745) (end 151.638 116.205) (width 1) (layer F.Cu) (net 35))
 (segment (start 159.258 118.745) (end 154.178 118.745) (width 1) (layer F.Cu) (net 35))
 (segment (start 151.638 116.205) (end 149.098 116.205) (width 1) (layer B.Cu) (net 35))
 (segment (start 149.098 116.205) (end 146.558 113.665) (width 1) (layer B.Cu) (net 35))
 (segment (start 146.558 113.665) (end 136.398 113.665) (width 1) (layer B.Cu) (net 35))
 (segment (start 136.398 113.665) (end 135.128 112.395) (width 1) (layer B.Cu) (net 35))
 (segment (start 135.128 112.395) (end 135.128 109.855) (width 1) (layer B.Cu) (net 35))
 (segment (start 136.398 108.585) (end 138.938 108.585) (width 1) (layer B.Cu) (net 35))
 (segment (start 135.128 109.855) (end 136.398 108.585) (width 1) (layer B.Cu) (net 35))
 (segment (start 151.638 114.305) (end 153.538 116.205) (width 1) (layer B.Cu) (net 36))
 (segment (start 151.638 109.855) (end 151.638 114.305) (width 1) (layer B.Cu) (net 36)))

